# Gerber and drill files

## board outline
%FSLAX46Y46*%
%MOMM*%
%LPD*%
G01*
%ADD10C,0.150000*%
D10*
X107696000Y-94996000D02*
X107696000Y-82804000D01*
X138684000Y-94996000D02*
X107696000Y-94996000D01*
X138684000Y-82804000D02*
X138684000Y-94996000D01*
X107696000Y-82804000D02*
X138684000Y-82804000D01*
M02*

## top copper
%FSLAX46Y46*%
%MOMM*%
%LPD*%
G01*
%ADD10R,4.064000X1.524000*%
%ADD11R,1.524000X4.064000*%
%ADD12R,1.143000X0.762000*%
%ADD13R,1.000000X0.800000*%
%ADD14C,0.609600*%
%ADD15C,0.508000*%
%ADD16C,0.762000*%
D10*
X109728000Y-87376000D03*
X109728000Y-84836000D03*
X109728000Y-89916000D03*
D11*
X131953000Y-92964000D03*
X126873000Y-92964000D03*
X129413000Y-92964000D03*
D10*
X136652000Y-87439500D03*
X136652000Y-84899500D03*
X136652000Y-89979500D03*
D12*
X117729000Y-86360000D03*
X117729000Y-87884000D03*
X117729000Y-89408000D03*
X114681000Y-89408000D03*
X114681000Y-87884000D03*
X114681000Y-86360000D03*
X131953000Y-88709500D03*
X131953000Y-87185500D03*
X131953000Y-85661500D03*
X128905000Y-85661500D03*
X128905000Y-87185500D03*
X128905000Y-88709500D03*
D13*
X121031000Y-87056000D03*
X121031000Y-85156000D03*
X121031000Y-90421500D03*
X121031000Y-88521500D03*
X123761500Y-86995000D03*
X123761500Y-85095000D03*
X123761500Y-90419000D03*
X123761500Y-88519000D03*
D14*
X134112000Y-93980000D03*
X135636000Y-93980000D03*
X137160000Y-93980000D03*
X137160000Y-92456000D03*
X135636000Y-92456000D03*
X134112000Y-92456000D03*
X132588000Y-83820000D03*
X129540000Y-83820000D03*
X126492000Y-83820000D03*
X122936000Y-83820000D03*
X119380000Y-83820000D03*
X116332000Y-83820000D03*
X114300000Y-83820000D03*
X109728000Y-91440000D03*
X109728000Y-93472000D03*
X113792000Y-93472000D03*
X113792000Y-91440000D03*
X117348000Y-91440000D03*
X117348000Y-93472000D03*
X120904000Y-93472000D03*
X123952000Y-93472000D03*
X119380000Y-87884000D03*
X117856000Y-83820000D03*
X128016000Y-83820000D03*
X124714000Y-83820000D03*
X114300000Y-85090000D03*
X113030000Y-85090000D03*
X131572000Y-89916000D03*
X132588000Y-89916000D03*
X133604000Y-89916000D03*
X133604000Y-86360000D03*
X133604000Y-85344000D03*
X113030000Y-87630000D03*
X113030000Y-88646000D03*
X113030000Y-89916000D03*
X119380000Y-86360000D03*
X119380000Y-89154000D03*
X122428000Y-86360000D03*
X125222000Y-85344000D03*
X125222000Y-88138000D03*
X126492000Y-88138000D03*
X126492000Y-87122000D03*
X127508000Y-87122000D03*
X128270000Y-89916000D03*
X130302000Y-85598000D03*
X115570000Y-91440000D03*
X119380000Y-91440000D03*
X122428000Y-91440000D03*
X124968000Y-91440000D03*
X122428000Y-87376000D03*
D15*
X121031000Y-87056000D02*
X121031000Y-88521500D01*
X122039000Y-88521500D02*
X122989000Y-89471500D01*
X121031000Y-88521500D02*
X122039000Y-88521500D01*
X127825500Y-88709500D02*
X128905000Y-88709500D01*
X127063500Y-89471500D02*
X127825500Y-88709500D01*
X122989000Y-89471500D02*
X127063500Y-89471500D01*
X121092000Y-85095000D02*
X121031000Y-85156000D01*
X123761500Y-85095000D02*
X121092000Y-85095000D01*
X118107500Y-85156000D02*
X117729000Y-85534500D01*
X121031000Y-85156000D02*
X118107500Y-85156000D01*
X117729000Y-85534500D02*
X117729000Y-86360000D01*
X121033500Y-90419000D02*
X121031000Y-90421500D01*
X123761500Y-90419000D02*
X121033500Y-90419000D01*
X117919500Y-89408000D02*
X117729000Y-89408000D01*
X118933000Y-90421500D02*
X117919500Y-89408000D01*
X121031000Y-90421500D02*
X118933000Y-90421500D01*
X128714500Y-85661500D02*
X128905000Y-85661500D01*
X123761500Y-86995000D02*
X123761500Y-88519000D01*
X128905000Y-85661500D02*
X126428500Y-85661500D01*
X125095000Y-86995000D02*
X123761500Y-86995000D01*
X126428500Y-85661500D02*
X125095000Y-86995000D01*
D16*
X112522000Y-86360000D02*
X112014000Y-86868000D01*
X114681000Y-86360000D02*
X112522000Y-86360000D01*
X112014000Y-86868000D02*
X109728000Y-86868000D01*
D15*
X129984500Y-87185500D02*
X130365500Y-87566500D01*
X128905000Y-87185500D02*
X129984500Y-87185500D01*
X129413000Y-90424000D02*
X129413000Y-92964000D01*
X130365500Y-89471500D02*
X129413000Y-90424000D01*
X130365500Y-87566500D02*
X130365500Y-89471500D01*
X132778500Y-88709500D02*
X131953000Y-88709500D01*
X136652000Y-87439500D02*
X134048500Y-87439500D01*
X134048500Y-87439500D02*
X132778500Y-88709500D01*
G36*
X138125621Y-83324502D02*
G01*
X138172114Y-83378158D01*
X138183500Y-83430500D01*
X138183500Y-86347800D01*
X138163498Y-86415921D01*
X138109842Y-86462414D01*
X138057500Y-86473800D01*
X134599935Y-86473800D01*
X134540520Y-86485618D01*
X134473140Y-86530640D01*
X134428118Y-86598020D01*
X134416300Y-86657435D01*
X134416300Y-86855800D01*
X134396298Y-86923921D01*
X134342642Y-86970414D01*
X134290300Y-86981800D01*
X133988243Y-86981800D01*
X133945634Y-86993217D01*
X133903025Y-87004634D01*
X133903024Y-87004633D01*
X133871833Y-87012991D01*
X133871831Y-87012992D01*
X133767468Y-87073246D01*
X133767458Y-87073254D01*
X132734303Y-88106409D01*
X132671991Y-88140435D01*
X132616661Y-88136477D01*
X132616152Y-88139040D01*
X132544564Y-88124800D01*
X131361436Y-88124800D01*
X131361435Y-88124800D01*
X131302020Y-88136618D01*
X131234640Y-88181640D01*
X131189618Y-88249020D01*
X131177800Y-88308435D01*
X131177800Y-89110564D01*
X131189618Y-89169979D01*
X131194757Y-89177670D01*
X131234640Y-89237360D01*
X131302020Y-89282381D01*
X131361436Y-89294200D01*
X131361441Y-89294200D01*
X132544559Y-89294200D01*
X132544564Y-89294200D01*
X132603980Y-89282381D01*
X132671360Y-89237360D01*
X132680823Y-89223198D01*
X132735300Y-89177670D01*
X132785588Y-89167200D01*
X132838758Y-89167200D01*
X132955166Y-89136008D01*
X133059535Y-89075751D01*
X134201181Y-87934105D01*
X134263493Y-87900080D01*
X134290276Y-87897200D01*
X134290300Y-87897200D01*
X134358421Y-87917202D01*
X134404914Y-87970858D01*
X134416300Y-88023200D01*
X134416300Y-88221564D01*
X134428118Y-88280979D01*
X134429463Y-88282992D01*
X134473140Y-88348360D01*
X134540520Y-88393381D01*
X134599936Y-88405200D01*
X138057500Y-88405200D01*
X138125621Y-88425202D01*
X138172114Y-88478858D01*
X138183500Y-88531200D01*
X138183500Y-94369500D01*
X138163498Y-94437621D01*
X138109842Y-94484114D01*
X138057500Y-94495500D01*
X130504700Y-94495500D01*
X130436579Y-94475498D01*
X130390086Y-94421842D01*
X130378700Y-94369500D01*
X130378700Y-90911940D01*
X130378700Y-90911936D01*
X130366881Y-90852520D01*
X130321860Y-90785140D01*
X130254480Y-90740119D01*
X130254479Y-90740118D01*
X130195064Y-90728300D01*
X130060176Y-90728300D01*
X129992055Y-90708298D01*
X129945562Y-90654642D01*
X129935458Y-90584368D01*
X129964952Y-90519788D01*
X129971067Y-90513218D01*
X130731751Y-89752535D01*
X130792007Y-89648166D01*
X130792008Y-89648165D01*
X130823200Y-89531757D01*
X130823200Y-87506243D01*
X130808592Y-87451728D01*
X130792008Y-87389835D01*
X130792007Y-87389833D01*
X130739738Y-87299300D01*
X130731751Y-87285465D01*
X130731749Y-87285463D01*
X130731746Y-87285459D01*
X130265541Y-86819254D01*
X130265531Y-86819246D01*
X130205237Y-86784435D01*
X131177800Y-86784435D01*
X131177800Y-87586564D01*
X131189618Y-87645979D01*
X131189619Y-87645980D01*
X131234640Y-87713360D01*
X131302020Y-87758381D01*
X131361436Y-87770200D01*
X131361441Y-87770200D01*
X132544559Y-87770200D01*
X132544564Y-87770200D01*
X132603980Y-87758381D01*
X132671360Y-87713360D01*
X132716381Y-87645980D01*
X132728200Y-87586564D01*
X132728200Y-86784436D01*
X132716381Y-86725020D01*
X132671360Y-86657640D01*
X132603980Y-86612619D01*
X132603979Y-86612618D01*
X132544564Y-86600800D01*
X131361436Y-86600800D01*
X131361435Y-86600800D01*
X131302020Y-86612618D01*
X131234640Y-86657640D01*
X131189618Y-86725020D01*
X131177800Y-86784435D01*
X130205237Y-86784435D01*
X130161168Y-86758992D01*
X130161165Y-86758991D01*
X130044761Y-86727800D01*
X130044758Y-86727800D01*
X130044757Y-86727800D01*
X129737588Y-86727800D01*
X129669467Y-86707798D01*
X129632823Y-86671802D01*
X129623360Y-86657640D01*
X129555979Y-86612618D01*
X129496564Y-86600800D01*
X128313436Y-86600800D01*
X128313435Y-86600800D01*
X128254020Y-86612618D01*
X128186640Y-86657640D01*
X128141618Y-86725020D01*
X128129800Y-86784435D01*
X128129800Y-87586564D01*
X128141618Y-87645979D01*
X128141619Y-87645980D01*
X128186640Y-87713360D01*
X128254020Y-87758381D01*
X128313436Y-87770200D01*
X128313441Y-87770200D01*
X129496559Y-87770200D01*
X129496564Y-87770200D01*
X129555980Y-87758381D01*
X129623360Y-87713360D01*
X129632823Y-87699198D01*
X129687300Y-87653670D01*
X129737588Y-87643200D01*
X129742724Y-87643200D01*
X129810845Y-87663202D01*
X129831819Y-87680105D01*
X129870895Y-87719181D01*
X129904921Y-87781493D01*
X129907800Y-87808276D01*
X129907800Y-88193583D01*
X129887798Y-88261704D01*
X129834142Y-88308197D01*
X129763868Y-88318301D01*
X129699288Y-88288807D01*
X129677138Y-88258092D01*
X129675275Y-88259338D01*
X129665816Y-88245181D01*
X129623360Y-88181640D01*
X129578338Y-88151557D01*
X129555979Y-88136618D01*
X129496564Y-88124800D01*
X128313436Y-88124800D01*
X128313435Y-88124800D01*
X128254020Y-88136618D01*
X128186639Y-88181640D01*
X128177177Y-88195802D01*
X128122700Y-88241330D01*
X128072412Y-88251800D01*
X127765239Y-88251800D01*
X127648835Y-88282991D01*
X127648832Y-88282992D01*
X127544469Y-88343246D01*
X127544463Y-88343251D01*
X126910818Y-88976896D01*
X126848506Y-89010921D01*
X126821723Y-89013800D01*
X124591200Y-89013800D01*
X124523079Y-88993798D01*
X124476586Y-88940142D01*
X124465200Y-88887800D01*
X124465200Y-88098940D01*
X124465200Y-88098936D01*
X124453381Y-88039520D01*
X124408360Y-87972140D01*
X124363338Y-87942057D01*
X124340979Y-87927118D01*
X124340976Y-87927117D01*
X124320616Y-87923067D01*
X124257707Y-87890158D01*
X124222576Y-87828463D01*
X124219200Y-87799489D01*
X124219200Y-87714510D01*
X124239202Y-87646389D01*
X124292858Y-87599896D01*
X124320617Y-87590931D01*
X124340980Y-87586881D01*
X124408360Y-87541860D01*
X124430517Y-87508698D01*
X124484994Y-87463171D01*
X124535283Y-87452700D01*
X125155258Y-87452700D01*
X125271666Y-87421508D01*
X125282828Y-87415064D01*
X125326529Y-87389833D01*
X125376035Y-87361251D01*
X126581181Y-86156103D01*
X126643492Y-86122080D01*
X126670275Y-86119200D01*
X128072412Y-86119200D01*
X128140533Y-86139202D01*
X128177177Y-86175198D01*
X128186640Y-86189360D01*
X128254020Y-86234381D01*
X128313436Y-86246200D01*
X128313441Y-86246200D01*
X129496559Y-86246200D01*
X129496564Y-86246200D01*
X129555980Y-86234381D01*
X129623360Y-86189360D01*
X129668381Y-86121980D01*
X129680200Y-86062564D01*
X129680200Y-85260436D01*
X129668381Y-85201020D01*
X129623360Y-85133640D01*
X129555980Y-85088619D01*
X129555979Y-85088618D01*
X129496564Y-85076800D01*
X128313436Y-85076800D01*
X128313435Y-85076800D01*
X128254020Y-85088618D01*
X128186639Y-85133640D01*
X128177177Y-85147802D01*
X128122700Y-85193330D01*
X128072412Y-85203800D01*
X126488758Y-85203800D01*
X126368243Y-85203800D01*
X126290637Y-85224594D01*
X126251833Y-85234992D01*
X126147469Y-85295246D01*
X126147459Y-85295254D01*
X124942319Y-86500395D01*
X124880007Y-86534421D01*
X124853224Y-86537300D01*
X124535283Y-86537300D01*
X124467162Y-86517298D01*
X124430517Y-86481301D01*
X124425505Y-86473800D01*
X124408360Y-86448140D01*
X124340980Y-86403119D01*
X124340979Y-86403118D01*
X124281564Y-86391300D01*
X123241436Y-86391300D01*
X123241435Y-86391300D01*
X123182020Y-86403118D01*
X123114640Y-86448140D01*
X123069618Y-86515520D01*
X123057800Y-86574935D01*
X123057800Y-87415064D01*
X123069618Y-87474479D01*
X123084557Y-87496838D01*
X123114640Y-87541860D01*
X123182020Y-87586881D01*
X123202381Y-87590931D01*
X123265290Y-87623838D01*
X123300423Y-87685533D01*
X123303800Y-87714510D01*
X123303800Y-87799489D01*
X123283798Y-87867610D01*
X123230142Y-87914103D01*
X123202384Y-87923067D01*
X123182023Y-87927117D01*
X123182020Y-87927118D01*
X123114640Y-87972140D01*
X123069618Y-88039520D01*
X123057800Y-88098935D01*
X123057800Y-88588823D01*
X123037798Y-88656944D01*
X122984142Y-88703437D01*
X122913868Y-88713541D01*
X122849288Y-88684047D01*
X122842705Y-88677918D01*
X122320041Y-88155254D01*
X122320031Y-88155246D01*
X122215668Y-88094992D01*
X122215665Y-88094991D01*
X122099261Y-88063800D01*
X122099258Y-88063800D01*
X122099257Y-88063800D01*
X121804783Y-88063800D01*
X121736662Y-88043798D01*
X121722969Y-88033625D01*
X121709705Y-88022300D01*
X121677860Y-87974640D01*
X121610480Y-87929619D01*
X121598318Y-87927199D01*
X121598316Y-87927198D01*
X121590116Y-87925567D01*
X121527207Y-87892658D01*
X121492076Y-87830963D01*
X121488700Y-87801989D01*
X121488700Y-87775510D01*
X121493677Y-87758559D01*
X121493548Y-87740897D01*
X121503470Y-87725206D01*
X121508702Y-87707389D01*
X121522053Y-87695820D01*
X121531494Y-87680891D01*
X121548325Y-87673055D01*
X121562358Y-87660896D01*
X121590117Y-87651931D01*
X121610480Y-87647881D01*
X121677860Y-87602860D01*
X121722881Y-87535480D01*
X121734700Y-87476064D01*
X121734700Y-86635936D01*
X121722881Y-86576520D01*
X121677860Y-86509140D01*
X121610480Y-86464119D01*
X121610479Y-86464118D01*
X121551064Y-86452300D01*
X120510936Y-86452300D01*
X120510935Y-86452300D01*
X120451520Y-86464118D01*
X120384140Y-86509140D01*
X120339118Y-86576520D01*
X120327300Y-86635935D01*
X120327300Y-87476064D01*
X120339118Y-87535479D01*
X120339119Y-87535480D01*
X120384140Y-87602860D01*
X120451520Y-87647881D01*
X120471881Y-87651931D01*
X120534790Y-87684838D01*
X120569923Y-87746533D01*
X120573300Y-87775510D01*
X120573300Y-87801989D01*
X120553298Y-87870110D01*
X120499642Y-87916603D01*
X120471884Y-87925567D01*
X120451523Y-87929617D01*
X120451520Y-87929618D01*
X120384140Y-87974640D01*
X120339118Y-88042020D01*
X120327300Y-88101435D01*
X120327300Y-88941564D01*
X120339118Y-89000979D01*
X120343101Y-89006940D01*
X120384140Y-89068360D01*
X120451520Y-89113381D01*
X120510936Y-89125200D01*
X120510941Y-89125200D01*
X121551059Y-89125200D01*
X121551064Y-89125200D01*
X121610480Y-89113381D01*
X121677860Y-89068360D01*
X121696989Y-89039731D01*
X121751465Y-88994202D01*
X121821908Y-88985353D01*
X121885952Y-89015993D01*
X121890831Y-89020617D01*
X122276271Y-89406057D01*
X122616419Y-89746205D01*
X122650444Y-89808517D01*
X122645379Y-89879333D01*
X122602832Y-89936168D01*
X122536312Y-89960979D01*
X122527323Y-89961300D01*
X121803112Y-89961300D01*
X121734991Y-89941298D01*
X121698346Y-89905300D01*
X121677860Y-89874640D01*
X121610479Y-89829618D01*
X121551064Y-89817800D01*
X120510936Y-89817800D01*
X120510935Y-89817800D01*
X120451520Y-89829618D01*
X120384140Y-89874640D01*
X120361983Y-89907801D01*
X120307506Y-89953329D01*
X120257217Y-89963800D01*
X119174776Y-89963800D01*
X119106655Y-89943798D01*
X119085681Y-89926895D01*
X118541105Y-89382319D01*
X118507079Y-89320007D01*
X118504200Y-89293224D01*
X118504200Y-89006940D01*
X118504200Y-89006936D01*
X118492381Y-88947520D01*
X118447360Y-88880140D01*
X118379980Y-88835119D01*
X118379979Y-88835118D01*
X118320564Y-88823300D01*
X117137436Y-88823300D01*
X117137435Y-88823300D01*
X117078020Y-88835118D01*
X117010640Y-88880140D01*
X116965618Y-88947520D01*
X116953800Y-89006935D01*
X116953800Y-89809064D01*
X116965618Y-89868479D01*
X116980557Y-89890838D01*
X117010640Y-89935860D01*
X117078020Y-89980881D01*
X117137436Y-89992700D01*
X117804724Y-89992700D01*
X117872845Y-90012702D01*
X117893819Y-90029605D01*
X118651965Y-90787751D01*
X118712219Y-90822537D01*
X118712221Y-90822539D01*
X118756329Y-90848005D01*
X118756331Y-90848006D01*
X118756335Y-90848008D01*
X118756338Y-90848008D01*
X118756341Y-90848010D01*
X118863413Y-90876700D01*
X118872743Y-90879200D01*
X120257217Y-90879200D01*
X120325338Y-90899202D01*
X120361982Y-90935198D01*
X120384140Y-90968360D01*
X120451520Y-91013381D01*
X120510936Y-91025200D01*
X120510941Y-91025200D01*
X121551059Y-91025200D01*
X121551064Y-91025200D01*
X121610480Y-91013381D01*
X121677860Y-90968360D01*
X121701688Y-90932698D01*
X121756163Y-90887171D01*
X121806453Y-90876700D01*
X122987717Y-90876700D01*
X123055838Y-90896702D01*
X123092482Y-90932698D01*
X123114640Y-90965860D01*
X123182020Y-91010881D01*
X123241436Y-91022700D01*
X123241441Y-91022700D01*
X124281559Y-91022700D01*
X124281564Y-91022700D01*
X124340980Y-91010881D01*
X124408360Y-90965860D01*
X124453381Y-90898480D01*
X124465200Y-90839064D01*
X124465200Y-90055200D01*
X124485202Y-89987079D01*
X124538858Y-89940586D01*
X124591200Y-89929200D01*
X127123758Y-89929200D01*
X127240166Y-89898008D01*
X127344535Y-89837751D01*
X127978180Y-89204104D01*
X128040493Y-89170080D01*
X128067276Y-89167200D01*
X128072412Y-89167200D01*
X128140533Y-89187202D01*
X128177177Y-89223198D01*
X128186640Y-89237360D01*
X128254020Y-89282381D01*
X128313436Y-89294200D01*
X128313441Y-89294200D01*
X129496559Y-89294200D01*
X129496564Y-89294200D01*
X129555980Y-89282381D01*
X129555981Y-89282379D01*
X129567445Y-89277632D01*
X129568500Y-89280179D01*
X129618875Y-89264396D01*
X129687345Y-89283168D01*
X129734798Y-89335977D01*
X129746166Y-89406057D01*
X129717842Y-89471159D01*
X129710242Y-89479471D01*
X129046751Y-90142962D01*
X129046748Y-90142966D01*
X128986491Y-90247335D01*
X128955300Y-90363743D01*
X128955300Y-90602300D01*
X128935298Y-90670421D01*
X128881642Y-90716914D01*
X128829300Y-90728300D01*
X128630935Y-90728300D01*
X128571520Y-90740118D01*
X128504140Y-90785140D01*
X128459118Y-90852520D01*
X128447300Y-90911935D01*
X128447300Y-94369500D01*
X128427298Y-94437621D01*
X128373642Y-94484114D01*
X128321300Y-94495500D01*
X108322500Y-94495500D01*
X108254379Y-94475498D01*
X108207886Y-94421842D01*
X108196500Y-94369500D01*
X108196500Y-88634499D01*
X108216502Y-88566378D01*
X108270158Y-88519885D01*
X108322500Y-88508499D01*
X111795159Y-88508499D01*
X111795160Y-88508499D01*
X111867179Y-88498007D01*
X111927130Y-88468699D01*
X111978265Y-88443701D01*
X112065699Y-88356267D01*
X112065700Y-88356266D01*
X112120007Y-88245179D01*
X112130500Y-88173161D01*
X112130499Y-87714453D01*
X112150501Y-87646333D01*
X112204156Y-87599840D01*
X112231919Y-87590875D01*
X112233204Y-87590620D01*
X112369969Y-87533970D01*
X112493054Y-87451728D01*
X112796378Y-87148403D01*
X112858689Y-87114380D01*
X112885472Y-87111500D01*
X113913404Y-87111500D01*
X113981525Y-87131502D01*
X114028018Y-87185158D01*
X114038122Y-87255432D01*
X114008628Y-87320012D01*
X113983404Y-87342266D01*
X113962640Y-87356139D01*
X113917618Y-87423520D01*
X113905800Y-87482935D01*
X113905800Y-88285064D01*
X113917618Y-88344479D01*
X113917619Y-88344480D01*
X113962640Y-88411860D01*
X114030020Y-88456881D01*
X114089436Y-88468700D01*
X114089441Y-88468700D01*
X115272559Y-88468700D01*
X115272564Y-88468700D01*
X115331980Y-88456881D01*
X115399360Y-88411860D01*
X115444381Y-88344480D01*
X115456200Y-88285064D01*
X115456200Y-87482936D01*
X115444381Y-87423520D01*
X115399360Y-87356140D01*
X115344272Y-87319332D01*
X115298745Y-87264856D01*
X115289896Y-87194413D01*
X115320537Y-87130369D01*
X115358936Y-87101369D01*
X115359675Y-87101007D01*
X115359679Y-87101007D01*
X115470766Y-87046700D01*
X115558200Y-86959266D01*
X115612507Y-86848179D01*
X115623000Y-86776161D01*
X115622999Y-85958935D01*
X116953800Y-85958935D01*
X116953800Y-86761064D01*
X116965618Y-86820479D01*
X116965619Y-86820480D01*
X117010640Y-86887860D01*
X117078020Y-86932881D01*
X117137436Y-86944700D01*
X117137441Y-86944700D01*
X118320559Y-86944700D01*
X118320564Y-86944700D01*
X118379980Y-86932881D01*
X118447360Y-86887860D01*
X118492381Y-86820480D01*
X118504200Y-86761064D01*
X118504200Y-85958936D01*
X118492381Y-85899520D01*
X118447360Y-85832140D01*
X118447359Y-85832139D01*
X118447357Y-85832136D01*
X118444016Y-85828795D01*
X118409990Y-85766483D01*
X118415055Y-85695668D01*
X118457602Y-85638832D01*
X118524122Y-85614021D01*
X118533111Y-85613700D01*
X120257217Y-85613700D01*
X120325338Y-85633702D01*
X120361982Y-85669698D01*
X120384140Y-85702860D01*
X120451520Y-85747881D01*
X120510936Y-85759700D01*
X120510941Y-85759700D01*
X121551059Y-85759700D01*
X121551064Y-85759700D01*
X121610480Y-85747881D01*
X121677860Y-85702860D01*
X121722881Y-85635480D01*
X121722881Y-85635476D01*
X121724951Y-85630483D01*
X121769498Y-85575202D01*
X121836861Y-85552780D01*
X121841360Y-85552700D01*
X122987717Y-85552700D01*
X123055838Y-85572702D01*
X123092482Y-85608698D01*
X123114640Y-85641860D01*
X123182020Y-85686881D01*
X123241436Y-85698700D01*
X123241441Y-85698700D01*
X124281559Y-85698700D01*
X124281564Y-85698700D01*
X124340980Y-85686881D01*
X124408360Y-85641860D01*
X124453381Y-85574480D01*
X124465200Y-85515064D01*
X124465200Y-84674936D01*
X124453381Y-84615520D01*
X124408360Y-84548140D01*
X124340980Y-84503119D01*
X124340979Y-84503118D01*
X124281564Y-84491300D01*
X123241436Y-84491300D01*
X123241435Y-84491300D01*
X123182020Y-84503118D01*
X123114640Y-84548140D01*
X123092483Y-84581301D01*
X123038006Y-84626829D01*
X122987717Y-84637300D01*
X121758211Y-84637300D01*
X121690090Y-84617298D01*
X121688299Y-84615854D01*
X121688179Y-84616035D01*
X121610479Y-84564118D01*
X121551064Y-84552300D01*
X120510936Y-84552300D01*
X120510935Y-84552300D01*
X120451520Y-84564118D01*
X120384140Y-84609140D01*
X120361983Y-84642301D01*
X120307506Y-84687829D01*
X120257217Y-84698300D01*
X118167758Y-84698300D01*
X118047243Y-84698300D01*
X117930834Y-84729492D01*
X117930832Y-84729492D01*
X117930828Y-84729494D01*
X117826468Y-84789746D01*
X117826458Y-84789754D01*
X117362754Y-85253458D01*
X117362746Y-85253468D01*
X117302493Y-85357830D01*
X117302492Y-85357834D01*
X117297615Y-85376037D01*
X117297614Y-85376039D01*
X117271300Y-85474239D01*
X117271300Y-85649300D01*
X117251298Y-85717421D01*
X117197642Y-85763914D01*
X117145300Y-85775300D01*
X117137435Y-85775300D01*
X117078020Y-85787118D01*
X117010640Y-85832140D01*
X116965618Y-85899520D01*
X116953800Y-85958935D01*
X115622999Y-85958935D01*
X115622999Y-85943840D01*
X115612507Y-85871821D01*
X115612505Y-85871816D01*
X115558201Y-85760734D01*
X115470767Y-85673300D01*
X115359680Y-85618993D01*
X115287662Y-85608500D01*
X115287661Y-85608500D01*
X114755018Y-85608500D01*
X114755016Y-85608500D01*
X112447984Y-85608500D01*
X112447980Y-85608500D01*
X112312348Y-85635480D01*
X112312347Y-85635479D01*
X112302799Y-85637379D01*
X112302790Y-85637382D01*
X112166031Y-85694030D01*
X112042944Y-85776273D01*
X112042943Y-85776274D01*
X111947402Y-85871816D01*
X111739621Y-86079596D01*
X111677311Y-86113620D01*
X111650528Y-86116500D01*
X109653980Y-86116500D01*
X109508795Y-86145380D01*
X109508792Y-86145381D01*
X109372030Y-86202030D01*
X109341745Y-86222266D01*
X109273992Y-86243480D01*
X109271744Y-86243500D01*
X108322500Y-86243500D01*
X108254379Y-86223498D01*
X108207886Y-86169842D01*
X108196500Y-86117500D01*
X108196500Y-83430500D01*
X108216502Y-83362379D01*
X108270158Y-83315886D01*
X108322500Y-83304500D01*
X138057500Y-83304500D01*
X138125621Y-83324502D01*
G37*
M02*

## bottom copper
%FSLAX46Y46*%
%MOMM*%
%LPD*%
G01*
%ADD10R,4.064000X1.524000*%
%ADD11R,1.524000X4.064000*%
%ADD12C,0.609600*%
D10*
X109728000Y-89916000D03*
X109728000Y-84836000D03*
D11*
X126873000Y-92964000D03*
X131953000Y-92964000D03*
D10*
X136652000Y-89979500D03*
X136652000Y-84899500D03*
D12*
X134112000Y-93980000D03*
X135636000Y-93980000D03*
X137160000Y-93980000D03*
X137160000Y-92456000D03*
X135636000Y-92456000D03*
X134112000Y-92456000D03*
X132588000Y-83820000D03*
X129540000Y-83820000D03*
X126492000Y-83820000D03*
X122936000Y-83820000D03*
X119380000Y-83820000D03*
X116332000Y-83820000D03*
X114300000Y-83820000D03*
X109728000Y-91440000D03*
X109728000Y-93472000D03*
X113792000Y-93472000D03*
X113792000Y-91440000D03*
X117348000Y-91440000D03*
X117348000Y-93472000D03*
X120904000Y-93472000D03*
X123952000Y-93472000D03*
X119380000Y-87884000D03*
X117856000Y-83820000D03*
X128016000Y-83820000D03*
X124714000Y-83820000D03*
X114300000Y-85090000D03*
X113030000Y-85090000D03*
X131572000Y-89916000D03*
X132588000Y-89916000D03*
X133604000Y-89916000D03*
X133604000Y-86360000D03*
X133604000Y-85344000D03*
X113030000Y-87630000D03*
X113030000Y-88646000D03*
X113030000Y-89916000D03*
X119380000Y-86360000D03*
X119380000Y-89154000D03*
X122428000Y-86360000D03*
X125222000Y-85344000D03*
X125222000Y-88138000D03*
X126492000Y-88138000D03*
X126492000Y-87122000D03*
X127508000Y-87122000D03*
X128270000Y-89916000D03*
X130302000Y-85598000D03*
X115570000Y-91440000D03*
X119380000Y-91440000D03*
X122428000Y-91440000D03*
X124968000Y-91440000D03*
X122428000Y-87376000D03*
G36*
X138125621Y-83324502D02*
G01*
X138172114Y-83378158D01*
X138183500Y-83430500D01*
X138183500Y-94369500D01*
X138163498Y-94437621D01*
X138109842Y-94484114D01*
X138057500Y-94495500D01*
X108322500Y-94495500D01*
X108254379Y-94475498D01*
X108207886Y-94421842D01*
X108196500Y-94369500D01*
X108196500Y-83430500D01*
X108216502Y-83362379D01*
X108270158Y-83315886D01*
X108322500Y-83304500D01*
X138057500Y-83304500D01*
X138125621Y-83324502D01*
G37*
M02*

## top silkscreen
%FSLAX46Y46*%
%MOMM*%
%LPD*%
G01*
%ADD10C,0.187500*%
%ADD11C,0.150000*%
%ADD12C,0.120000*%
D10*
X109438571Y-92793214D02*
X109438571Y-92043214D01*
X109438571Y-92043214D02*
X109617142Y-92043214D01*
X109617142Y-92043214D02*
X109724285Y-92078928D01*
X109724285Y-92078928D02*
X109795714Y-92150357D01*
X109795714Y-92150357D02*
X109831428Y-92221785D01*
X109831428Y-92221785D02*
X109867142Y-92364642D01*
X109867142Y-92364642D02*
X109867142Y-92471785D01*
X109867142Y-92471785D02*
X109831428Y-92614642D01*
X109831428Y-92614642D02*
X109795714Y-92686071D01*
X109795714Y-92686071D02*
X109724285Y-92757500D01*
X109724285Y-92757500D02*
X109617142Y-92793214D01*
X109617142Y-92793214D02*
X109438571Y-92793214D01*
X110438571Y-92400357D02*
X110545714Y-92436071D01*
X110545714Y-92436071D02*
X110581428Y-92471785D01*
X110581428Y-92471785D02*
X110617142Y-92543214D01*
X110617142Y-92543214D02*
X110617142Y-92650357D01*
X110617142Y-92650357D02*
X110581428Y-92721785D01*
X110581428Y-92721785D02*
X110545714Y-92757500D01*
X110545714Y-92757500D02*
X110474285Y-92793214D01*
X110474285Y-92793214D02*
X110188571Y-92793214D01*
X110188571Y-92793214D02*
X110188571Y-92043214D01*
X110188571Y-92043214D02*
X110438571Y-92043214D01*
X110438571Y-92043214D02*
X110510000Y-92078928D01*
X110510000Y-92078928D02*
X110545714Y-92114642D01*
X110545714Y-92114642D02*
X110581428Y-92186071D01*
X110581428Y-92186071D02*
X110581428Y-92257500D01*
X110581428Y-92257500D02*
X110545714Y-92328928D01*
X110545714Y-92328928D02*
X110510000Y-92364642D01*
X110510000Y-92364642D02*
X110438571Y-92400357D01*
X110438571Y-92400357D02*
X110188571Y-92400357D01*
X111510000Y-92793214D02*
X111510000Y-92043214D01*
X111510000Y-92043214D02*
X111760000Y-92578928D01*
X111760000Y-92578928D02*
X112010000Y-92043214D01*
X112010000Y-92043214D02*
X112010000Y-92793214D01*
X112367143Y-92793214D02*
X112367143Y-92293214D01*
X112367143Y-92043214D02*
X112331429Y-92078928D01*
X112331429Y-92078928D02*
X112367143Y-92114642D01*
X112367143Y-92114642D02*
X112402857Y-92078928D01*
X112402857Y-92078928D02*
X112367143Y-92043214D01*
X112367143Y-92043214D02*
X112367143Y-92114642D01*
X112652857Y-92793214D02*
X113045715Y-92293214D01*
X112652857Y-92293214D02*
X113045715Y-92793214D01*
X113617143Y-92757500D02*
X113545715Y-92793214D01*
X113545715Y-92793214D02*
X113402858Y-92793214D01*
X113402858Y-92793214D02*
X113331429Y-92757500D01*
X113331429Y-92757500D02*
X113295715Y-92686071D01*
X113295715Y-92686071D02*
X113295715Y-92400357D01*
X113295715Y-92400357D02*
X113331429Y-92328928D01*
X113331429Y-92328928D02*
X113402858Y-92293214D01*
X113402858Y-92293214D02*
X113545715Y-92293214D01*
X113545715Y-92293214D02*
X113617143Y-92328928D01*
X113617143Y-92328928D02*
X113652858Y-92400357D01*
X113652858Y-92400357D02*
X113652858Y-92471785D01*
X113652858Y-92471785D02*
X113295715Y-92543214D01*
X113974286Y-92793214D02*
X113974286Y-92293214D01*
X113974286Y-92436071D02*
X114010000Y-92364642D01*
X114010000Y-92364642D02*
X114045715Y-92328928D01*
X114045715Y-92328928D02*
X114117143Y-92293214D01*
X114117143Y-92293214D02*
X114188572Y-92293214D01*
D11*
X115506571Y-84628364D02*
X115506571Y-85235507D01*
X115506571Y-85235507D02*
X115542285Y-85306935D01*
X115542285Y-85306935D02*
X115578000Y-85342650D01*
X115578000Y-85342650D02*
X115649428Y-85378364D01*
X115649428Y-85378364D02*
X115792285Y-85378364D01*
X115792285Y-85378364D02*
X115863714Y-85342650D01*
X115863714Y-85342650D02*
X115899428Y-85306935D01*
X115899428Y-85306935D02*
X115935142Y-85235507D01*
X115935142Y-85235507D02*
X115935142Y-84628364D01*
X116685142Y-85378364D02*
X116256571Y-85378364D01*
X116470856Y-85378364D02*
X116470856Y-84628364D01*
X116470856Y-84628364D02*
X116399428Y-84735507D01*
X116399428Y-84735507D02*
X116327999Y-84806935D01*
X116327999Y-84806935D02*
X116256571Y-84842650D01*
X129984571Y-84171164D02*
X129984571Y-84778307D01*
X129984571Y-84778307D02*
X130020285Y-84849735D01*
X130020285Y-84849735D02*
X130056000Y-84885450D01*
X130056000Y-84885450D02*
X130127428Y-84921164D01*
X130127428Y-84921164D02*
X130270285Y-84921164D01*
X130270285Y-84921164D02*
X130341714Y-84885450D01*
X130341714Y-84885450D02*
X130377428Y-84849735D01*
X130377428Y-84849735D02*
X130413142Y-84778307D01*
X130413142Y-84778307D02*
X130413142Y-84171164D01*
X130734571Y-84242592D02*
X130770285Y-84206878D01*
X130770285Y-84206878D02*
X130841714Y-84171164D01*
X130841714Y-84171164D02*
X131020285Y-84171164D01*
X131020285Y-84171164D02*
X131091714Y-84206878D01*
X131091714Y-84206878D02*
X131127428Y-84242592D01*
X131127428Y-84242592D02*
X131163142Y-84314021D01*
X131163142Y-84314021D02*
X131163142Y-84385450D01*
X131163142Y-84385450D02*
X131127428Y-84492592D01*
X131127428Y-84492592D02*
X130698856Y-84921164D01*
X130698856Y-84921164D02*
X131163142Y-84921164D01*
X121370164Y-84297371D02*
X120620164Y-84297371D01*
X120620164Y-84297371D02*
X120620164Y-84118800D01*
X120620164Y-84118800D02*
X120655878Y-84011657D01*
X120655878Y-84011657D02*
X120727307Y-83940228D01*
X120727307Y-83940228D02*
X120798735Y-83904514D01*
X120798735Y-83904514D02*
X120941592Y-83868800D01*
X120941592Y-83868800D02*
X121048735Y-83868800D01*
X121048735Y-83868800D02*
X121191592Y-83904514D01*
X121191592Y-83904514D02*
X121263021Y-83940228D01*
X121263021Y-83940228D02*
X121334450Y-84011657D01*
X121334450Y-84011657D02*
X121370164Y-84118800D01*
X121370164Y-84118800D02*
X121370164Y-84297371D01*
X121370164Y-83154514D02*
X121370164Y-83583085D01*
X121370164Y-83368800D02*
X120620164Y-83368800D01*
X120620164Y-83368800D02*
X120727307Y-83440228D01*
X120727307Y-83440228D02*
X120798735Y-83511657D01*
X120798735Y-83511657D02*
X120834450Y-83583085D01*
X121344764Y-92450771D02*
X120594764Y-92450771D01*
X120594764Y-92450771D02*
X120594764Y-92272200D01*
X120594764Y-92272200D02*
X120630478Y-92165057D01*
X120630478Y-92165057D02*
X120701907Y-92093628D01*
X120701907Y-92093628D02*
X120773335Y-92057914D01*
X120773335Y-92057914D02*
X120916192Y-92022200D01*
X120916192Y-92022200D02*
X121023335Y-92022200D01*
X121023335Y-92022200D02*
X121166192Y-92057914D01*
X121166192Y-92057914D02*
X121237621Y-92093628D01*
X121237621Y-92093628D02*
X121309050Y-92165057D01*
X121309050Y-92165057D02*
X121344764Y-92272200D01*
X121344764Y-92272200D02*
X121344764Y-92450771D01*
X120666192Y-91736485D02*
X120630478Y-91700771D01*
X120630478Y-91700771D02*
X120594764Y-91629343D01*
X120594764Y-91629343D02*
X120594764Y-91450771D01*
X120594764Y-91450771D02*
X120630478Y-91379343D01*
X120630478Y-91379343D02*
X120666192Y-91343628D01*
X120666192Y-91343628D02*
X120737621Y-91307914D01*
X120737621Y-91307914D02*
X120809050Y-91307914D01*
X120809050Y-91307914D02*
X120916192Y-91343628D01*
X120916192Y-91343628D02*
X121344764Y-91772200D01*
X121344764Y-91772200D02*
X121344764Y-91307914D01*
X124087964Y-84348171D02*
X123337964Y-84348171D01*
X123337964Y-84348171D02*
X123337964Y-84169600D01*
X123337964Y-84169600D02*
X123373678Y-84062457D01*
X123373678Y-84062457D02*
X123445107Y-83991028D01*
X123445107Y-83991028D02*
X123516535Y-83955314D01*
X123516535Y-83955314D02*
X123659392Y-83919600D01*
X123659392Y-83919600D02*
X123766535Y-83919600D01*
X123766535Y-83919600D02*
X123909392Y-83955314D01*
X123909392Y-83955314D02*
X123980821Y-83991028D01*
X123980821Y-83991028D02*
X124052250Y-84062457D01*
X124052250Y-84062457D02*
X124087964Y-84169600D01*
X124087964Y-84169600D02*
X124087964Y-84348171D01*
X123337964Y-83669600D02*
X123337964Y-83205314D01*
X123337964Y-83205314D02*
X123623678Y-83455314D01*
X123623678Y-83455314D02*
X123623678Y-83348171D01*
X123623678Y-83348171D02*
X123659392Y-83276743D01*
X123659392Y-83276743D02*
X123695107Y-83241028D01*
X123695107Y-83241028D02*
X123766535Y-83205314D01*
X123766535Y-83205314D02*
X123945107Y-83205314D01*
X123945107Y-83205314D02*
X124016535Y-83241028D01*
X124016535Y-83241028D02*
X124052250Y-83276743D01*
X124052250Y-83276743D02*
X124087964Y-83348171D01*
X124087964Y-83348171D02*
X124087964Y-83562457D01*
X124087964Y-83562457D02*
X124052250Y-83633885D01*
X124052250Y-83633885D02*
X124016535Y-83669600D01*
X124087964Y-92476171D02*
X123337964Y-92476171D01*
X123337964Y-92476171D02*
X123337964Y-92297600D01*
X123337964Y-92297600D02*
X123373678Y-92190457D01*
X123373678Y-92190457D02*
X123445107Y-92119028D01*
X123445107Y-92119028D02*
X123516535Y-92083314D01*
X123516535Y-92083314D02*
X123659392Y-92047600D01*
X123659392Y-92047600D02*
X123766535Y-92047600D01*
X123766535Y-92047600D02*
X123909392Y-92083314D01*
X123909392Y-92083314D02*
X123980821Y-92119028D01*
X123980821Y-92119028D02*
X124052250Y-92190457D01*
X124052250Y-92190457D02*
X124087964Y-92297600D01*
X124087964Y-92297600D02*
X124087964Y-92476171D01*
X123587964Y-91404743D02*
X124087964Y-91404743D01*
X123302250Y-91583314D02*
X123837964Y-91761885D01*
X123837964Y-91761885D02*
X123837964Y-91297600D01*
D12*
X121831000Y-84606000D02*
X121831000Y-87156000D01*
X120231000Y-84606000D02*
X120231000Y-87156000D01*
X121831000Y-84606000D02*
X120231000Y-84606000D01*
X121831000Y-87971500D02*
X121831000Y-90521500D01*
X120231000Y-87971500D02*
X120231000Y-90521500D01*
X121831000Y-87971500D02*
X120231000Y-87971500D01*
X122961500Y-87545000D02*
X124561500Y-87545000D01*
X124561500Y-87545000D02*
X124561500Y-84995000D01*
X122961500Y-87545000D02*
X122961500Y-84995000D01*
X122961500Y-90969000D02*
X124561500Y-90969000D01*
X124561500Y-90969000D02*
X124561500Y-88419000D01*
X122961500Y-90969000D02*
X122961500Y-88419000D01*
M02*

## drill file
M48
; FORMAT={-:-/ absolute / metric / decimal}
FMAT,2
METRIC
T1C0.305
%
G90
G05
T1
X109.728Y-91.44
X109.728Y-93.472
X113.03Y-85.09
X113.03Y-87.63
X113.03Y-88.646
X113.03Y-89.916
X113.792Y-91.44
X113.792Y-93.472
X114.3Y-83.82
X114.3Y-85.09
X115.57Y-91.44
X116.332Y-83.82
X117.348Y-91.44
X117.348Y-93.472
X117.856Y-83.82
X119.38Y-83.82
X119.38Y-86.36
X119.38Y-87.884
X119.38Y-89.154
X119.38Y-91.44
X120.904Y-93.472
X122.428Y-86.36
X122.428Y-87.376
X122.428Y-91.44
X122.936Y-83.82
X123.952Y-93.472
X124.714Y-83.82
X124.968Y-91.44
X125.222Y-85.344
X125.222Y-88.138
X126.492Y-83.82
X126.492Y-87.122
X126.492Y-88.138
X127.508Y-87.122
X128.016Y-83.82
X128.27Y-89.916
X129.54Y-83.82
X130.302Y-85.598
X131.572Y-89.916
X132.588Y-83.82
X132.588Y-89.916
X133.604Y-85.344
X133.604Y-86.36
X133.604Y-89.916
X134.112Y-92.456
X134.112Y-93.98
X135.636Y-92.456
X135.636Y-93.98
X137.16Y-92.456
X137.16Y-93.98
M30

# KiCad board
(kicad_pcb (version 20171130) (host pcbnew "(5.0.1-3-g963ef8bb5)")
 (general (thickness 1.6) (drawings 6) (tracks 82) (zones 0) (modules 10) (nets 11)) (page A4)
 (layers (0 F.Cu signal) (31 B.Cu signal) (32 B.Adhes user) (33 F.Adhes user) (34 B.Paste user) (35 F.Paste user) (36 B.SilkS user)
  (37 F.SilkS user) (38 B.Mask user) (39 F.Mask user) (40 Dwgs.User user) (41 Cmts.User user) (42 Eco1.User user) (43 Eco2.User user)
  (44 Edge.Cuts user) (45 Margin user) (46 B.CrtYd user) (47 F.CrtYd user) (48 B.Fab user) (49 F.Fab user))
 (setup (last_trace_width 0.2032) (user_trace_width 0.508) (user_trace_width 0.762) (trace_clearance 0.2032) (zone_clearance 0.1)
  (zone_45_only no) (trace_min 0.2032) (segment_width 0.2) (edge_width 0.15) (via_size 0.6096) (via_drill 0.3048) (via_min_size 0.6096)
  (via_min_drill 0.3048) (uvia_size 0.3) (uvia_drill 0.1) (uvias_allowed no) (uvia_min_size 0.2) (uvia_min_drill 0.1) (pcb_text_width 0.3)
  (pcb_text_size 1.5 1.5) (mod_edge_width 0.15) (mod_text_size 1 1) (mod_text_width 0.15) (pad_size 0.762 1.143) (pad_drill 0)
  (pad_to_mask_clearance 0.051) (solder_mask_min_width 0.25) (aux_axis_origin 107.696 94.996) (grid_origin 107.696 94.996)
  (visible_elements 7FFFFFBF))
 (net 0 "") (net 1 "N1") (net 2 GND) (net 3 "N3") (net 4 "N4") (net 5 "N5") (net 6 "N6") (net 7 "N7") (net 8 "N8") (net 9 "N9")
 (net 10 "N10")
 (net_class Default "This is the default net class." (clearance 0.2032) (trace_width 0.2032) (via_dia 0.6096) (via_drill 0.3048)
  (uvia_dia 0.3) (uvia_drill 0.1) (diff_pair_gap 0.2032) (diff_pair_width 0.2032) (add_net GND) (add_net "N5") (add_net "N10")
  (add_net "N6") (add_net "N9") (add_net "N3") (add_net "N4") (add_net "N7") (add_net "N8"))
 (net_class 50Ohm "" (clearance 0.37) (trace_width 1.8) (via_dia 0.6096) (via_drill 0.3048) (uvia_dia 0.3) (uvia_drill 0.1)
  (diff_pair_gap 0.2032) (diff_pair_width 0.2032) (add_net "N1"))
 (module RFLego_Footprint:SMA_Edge (layer F.Cu) (at 107.696 87.376)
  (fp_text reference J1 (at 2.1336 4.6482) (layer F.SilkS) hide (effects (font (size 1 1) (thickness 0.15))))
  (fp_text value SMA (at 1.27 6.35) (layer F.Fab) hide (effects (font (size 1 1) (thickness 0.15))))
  (pad 1 smd rect (at 2.032 0) (size 4.064 1.524) (layers F.Cu F.Mask) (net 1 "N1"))
  (pad 2 smd rect (at 2.032 -2.54) (size 4.064 1.524) (layers F.Cu F.Mask) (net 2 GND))
  (pad 2 smd rect (at 2.032 2.54) (size 4.064 1.524) (layers B.Cu B.Mask) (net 2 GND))
  (pad 2 smd rect (at 2.032 -2.54) (size 4.064 1.524) (layers B.Cu B.Mask) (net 2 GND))
  (pad 2 smd rect (at 2.032 2.54) (size 4.064 1.524) (layers F.Cu F.Mask) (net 2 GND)))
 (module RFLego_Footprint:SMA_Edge (layer F.Cu) (at 129.413 94.996 90)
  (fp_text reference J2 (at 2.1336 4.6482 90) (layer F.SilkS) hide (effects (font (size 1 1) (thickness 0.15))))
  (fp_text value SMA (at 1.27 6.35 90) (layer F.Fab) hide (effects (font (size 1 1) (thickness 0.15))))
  (pad 2 smd rect (at 2.032 2.54 90) (size 4.064 1.524) (layers F.Cu F.Mask) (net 2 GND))
  (pad 2 smd rect (at 2.032 -2.54 90) (size 4.064 1.524) (layers B.Cu B.Mask) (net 2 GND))
  (pad 2 smd rect (at 2.032 2.54 90) (size 4.064 1.524) (layers B.Cu B.Mask) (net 2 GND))
  (pad 2 smd rect (at 2.032 -2.54 90) (size 4.064 1.524) (layers F.Cu F.Mask) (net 2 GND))
  (pad 1 smd rect (at 2.032 0 90) (size 4.064 1.524) (layers F.Cu F.Mask) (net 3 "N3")))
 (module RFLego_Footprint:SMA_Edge (layer F.Cu) (at 134.62 87.4395)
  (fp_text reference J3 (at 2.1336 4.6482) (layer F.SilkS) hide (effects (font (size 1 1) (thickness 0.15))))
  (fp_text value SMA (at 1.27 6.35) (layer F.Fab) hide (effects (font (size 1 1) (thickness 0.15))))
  (pad 1 smd rect (at 2.032 0) (size 4.064 1.524) (layers F.Cu F.Mask) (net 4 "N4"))
  (pad 2 smd rect (at 2.032 -2.54) (size 4.064 1.524) (layers F.Cu F.Mask) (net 2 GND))
  (pad 2 smd rect (at 2.032 2.54) (size 4.064 1.524) (layers B.Cu B.Mask) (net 2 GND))
  (pad 2 smd rect (at 2.032 -2.54) (size 4.064 1.524) (layers B.Cu B.Mask) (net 2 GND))
  (pad 2 smd rect (at 2.032 2.54) (size 4.064 1.524) (layers F.Cu F.Mask) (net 2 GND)))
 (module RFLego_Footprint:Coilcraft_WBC (layer F.Cu) (at 117.729 86.36 270)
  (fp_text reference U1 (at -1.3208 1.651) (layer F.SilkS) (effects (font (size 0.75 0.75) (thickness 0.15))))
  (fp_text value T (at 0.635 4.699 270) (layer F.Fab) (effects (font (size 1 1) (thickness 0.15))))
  (pad 1 smd rect (at 0 0 270) (size 0.762 1.143) (layers F.Cu F.Paste F.Mask) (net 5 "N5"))
  (pad 2 smd rect (at 1.524 0 270) (size 0.762 1.143) (layers F.Cu F.Paste F.Mask) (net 2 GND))
  (pad 3 smd rect (at 3.048 0 270) (size 0.762 1.143) (layers F.Cu F.Paste F.Mask) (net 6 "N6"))
  (pad 4 smd rect (at 3.048 3.048 270) (size 0.762 1.143) (layers F.Cu F.Paste F.Mask) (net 2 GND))
  (pad 5 smd rect (at 1.524 3.048 270) (size 0.762 1.143) (layers F.Cu F.Paste F.Mask) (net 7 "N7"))
  (pad 6 smd rect (at 0 3.048 270) (size 0.762 1.143) (layers F.Cu F.Paste F.Mask) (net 1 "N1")))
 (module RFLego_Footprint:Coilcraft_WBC (layer F.Cu) (at 128.905 88.7095 90)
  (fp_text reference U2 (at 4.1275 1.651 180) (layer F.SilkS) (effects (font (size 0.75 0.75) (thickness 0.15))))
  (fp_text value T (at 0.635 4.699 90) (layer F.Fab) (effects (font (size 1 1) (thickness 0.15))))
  (pad 6 smd rect (at 0 3.048 90) (size 0.762 1.143) (layers F.Cu F.Paste F.Mask) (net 4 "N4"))
  (pad 5 smd rect (at 1.524 3.048 90) (size 0.762 1.143) (layers F.Cu F.Paste F.Mask) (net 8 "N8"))
  (pad 4 smd rect (at 3.048 3.048 90) (size 0.762 1.143) (layers F.Cu F.Paste F.Mask) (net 2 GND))
  (pad 3 smd rect (at 3.048 0 90) (size 0.762 1.143) (layers F.Cu F.Paste F.Mask) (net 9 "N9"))
  (pad 2 smd rect (at 1.524 0 90) (size 0.762 1.143) (layers F.Cu F.Paste F.Mask) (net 3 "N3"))
  (pad 1 smd rect (at 0 0 90) (size 0.762 1.143) (layers F.Cu F.Paste F.Mask) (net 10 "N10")))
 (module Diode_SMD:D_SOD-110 (layer F.Cu) (at 121.031 86.106 270)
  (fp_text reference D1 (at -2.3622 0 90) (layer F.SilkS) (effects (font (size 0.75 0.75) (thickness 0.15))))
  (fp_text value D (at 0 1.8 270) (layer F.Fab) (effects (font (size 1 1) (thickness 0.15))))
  (fp_line (start -1.5 -0.8) (end 1.05 -0.8) (layer F.SilkS) (width 0.12))
  (fp_line (start -1.5 0.8) (end 1.05 0.8) (layer F.SilkS) (width 0.12))
  (fp_line (start -1.5 -0.8) (end -1.5 0.8) (layer F.SilkS) (width 0.12))
  (pad 2 smd rect (at 0.95 0 270) (size 0.8 1) (layers F.Cu F.Paste F.Mask) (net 10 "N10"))
  (pad 1 smd rect (at -0.95 0 270) (size 0.8 1) (layers F.Cu F.Paste F.Mask) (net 5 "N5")))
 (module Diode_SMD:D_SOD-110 (layer F.Cu) (at 121.031 89.4715 270)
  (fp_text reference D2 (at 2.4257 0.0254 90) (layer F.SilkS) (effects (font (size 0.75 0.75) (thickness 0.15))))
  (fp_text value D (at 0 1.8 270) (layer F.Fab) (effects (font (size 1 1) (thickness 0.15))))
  (fp_line (start -1.5 -0.8) (end 1.05 -0.8) (layer F.SilkS) (width 0.12))
  (fp_line (start -1.5 0.8) (end 1.05 0.8) (layer F.SilkS) (width 0.12))
  (fp_line (start -1.5 -0.8) (end -1.5 0.8) (layer F.SilkS) (width 0.12))
  (pad 2 smd rect (at 0.95 0 270) (size 0.8 1) (layers F.Cu F.Paste F.Mask) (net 6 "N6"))
  (pad 1 smd rect (at -0.95 0 270) (size 0.8 1) (layers F.Cu F.Paste F.Mask) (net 10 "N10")))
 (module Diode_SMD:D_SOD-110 (layer F.Cu) (at 123.7615 86.045 90)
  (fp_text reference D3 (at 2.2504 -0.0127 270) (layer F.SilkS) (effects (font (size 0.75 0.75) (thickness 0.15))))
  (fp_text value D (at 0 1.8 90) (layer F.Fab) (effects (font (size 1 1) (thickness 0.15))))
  (fp_line (start -1.5 -0.8) (end -1.5 0.8) (layer F.SilkS) (width 0.12))
  (fp_line (start -1.5 0.8) (end 1.05 0.8) (layer F.SilkS) (width 0.12))
  (fp_line (start -1.5 -0.8) (end 1.05 -0.8) (layer F.SilkS) (width 0.12))
  (pad 1 smd rect (at -0.95 0 90) (size 0.8 1) (layers F.Cu F.Paste F.Mask) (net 9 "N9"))
  (pad 2 smd rect (at 0.95 0 90) (size 0.8 1) (layers F.Cu F.Paste F.Mask) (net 5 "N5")))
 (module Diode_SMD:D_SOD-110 (layer F.Cu) (at 123.7615 89.469 90)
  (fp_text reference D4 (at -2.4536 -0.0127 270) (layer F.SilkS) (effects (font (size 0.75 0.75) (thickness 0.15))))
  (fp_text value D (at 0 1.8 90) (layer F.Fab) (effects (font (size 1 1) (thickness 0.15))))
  (fp_line (start -1.5 -0.8) (end -1.5 0.8) (layer F.SilkS) (width 0.12))
  (fp_line (start -1.5 0.8) (end 1.05 0.8) (layer F.SilkS) (width 0.12))
  (fp_line (start -1.5 -0.8) (end 1.05 -0.8) (layer F.SilkS) (width 0.12))
  (pad 1 smd rect (at -0.95 0 90) (size 0.8 1) (layers F.Cu F.Paste F.Mask) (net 6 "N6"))
  (pad 2 smd rect (at 0.95 0 90) (size 0.8 1) (layers F.Cu F.Paste F.Mask) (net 9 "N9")))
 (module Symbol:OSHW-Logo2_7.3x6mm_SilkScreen (layer B.Cu) (at 129.54 87.376 180)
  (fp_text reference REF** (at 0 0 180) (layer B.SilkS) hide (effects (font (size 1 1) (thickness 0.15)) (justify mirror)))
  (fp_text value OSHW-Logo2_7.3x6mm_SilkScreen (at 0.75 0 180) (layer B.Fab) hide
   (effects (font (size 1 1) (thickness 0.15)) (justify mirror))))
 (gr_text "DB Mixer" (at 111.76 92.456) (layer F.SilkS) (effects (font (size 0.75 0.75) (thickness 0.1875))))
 (gr_line (start 107.696 94.996) (end 107.696 82.804) (layer Edge.Cuts) (width 0.15))
 (gr_line (start 138.684 94.996) (end 107.696 94.996) (layer Edge.Cuts) (width 0.15))
 (gr_line (start 138.684 82.804) (end 138.684 94.996) (layer Edge.Cuts) (width 0.15))
 (gr_line (start 107.696 82.804) (end 138.684 82.804) (layer Edge.Cuts) (width 0.15))
 (segment (start 121.031 87.056) (end 121.031 88.5215) (width 0.508) (layer F.Cu) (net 10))
 (segment (start 122.039 88.5215) (end 122.989 89.4715) (width 0.508) (layer F.Cu) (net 10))
 (segment (start 121.031 88.5215) (end 122.039 88.5215) (width 0.508) (layer F.Cu) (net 10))
 (segment (start 127.8255 88.7095) (end 128.905 88.7095) (width 0.508) (layer F.Cu) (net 10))
 (segment (start 127.0635 89.4715) (end 127.8255 88.7095) (width 0.508) (layer F.Cu) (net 10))
 (segment (start 122.989 89.4715) (end 127.0635 89.4715) (width 0.508) (layer F.Cu) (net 10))
 (segment (start 121.092 85.095) (end 121.031 85.156) (width 0.508) (layer F.Cu) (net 5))
 (segment (start 123.7615 85.095) (end 121.092 85.095) (width 0.508) (layer F.Cu) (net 5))
 (segment (start 118.1075 85.156) (end 117.729 85.5345) (width 0.508) (layer F.Cu) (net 5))
 (segment (start 121.031 85.156) (end 118.1075 85.156) (width 0.508) (layer F.Cu) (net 5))
 (segment (start 117.729 85.5345) (end 117.729 86.36) (width 0.508) (layer F.Cu) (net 5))
 (segment (start 121.0335 90.419) (end 121.031 90.4215) (width 0.508) (layer F.Cu) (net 6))
 (segment (start 123.7615 90.419) (end 121.0335 90.419) (width 0.508) (layer F.Cu) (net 6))
 (segment (start 117.9195 89.408) (end 117.729 89.408) (width 0.508) (layer F.Cu) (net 6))
 (segment (start 118.933 90.4215) (end 117.9195 89.408) (width 0.508) (layer F.Cu) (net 6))
 (segment (start 121.031 90.4215) (end 118.933 90.4215) (width 0.508) (layer F.Cu) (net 6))
 (segment (start 128.7145 85.6615) (end 128.905 85.6615) (width 0.508) (layer F.Cu) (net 9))
 (segment (start 123.7615 86.995) (end 123.7615 88.519) (width 0.508) (layer F.Cu) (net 9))
 (segment (start 128.905 85.6615) (end 126.4285 85.6615) (width 0.508) (layer F.Cu) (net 9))
 (segment (start 125.095 86.995) (end 123.7615 86.995) (width 0.508) (layer F.Cu) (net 9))
 (segment (start 126.4285 85.6615) (end 125.095 86.995) (width 0.508) (layer F.Cu) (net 9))
 (segment (start 112.522 86.36) (end 112.014 86.868) (width 0.762) (layer F.Cu) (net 1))
 (segment (start 114.681 86.36) (end 112.522 86.36) (width 0.762) (layer F.Cu) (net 1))
 (segment (start 112.014 86.868) (end 109.728 86.868) (width 0.762) (layer F.Cu) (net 1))
 (via (at 134.112 93.98) (size 0.6096) (drill 0.3048) (layers F.Cu B.Cu) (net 2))
 (via (at 135.636 93.98) (size 0.6096) (drill 0.3048) (layers F.Cu B.Cu) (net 2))
 (via (at 137.16 93.98) (size 0.6096) (drill 0.3048) (layers F.Cu B.Cu) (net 2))
 (via (at 137.16 92.456) (size 0.6096) (drill 0.3048) (layers F.Cu B.Cu) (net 2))
 (via (at 135.636 92.456) (size 0.6096) (drill 0.3048) (layers F.Cu B.Cu) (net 2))
 (via (at 134.112 92.456) (size 0.6096) (drill 0.3048) (layers F.Cu B.Cu) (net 2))
 (via (at 132.588 83.82) (size 0.6096) (drill 0.3048) (layers F.Cu B.Cu) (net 2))
 (via (at 129.54 83.82) (size 0.6096) (drill 0.3048) (layers F.Cu B.Cu) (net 2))
 (via (at 126.492 83.82) (size 0.6096) (drill 0.3048) (layers F.Cu B.Cu) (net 2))
 (via (at 122.936 83.82) (size 0.6096) (drill 0.3048) (layers F.Cu B.Cu) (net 2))
 (via (at 119.38 83.82) (size 0.6096) (drill 0.3048) (layers F.Cu B.Cu) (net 2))
 (via (at 116.332 83.82) (size 0.6096) (drill 0.3048) (layers F.Cu B.Cu) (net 2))
 (via (at 114.3 83.82) (size 0.6096) (drill 0.3048) (layers F.Cu B.Cu) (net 2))
 (via (at 109.728 91.44) (size 0.6096) (drill 0.3048) (layers F.Cu B.Cu) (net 2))
 (via (at 109.728 93.472) (size 0.6096) (drill 0.3048) (layers F.Cu B.Cu) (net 2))
 (via (at 113.792 93.472) (size 0.6096) (drill 0.3048) (layers F.Cu B.Cu) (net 2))
 (via (at 113.792 91.44) (size 0.6096) (drill 0.3048) (layers F.Cu B.Cu) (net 2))
 (via (at 117.348 91.44) (size 0.6096) (drill 0.3048) (layers F.Cu B.Cu) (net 2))
 (via (at 117.348 93.472) (size 0.6096) (drill 0.3048) (layers F.Cu B.Cu) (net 2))
 (via (at 120.904 93.472) (size 0.6096) (drill 0.3048) (layers F.Cu B.Cu) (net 2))
 (via (at 123.952 93.472) (size 0.6096) (drill 0.3048) (layers F.Cu B.Cu) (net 2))
 (via (at 119.38 87.884) (size 0.6096) (drill 0.3048) (layers F.Cu B.Cu) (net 2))
 (via (at 117.856 83.82) (size 0.6096) (drill 0.3048) (layers F.Cu B.Cu) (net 2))
 (via (at 128.016 83.82) (size 0.6096) (drill 0.3048) (layers F.Cu B.Cu) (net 2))
 (via (at 124.714 83.82) (size 0.6096) (drill 0.3048) (layers F.Cu B.Cu) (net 2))
 (via (at 114.3 85.09) (size 0.6096) (drill 0.3048) (layers F.Cu B.Cu) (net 2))
 (via (at 113.03 85.09) (size 0.6096) (drill 0.3048) (layers F.Cu B.Cu) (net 2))
 (via (at 131.572 89.916) (size 0.6096) (drill 0.3048) (layers F.Cu B.Cu) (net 2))
 (via (at 132.588 89.916) (size 0.6096) (drill 0.3048) (layers F.Cu B.Cu) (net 2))
 (via (at 133.604 89.916) (size 0.6096) (drill 0.3048) (layers F.Cu B.Cu) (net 2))
 (via (at 133.604 86.36) (size 0.6096) (drill 0.3048) (layers F.Cu B.Cu) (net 2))
 (via (at 133.604 85.344) (size 0.6096) (drill 0.3048) (layers F.Cu B.Cu) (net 2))
 (via (at 113.03 87.63) (size 0.6096) (drill 0.3048) (layers F.Cu B.Cu) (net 2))
 (via (at 113.03 88.646) (size 0.6096) (drill 0.3048) (layers F.Cu B.Cu) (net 2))
 (via (at 113.03 89.916) (size 0.6096) (drill 0.3048) (layers F.Cu B.Cu) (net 2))
 (via (at 119.38 86.36) (size 0.6096) (drill 0.3048) (layers F.Cu B.Cu) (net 2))
 (via (at 119.38 89.154) (size 0.6096) (drill 0.3048) (layers F.Cu B.Cu) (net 2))
 (via (at 122.428 86.36) (size 0.6096) (drill 0.3048) (layers F.Cu B.Cu) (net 2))
 (via (at 125.222 85.344) (size 0.6096) (drill 0.3048) (layers F.Cu B.Cu) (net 2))
 (via (at 125.222 88.138) (size 0.6096) (drill 0.3048) (layers F.Cu B.Cu) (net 2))
 (via (at 126.492 88.138) (size 0.6096) (drill 0.3048) (layers F.Cu B.Cu) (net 2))
 (via (at 126.492 87.122) (size 0.6096) (drill 0.3048) (layers F.Cu B.Cu) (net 2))
 (via (at 127.508 87.122) (size 0.6096) (drill 0.3048) (layers F.Cu B.Cu) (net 2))
 (via (at 128.27 89.916) (size 0.6096) (drill 0.3048) (layers F.Cu B.Cu) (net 2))
 (via (at 130.302 85.598) (size 0.6096) (drill 0.3048) (layers F.Cu B.Cu) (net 2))
 (via (at 115.57 91.44) (size 0.6096) (drill 0.3048) (layers F.Cu B.Cu) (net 2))
 (via (at 119.38 91.44) (size 0.6096) (drill 0.3048) (layers F.Cu B.Cu) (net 2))
 (via (at 122.428 91.44) (size 0.6096) (drill 0.3048) (layers F.Cu B.Cu) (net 2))
 (via (at 124.968 91.44) (size 0.6096) (drill 0.3048) (layers F.Cu B.Cu) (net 2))
 (via (at 122.428 87.376) (size 0.6096) (drill 0.3048) (layers F.Cu B.Cu) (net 2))
 (segment (start 129.9845 87.1855) (end 130.3655 87.5665) (width 0.508) (layer F.Cu) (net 3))
 (segment (start 128.905 87.1855) (end 129.9845 87.1855) (width 0.508) (layer F.Cu) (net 3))
 (segment (start 129.413 90.424) (end 129.413 92.964) (width 0.508) (layer F.Cu) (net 3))
 (segment (start 130.3655 89.4715) (end 129.413 90.424) (width 0.508) (layer F.Cu) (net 3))
 (segment (start 130.3655 87.5665) (end 130.3655 89.4715) (width 0.508) (layer F.Cu) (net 3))
 (segment (start 132.7785 88.7095) (end 131.953 88.7095) (width 0.508) (layer F.Cu) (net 4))
 (segment (start 136.652 87.4395) (end 134.0485 87.4395) (width 0.508) (layer F.Cu) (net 4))
 (segment (start 134.0485 87.4395) (end 132.7785 88.7095) (width 0.508) (layer F.Cu) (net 4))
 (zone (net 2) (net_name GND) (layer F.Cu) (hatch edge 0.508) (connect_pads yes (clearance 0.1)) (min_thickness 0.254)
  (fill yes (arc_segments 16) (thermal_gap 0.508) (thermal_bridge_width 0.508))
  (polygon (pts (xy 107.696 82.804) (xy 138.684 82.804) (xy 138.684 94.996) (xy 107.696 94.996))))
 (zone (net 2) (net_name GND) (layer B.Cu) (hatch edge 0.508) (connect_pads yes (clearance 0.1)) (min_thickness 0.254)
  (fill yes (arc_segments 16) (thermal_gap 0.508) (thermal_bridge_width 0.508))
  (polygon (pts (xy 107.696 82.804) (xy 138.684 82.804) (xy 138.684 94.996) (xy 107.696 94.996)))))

